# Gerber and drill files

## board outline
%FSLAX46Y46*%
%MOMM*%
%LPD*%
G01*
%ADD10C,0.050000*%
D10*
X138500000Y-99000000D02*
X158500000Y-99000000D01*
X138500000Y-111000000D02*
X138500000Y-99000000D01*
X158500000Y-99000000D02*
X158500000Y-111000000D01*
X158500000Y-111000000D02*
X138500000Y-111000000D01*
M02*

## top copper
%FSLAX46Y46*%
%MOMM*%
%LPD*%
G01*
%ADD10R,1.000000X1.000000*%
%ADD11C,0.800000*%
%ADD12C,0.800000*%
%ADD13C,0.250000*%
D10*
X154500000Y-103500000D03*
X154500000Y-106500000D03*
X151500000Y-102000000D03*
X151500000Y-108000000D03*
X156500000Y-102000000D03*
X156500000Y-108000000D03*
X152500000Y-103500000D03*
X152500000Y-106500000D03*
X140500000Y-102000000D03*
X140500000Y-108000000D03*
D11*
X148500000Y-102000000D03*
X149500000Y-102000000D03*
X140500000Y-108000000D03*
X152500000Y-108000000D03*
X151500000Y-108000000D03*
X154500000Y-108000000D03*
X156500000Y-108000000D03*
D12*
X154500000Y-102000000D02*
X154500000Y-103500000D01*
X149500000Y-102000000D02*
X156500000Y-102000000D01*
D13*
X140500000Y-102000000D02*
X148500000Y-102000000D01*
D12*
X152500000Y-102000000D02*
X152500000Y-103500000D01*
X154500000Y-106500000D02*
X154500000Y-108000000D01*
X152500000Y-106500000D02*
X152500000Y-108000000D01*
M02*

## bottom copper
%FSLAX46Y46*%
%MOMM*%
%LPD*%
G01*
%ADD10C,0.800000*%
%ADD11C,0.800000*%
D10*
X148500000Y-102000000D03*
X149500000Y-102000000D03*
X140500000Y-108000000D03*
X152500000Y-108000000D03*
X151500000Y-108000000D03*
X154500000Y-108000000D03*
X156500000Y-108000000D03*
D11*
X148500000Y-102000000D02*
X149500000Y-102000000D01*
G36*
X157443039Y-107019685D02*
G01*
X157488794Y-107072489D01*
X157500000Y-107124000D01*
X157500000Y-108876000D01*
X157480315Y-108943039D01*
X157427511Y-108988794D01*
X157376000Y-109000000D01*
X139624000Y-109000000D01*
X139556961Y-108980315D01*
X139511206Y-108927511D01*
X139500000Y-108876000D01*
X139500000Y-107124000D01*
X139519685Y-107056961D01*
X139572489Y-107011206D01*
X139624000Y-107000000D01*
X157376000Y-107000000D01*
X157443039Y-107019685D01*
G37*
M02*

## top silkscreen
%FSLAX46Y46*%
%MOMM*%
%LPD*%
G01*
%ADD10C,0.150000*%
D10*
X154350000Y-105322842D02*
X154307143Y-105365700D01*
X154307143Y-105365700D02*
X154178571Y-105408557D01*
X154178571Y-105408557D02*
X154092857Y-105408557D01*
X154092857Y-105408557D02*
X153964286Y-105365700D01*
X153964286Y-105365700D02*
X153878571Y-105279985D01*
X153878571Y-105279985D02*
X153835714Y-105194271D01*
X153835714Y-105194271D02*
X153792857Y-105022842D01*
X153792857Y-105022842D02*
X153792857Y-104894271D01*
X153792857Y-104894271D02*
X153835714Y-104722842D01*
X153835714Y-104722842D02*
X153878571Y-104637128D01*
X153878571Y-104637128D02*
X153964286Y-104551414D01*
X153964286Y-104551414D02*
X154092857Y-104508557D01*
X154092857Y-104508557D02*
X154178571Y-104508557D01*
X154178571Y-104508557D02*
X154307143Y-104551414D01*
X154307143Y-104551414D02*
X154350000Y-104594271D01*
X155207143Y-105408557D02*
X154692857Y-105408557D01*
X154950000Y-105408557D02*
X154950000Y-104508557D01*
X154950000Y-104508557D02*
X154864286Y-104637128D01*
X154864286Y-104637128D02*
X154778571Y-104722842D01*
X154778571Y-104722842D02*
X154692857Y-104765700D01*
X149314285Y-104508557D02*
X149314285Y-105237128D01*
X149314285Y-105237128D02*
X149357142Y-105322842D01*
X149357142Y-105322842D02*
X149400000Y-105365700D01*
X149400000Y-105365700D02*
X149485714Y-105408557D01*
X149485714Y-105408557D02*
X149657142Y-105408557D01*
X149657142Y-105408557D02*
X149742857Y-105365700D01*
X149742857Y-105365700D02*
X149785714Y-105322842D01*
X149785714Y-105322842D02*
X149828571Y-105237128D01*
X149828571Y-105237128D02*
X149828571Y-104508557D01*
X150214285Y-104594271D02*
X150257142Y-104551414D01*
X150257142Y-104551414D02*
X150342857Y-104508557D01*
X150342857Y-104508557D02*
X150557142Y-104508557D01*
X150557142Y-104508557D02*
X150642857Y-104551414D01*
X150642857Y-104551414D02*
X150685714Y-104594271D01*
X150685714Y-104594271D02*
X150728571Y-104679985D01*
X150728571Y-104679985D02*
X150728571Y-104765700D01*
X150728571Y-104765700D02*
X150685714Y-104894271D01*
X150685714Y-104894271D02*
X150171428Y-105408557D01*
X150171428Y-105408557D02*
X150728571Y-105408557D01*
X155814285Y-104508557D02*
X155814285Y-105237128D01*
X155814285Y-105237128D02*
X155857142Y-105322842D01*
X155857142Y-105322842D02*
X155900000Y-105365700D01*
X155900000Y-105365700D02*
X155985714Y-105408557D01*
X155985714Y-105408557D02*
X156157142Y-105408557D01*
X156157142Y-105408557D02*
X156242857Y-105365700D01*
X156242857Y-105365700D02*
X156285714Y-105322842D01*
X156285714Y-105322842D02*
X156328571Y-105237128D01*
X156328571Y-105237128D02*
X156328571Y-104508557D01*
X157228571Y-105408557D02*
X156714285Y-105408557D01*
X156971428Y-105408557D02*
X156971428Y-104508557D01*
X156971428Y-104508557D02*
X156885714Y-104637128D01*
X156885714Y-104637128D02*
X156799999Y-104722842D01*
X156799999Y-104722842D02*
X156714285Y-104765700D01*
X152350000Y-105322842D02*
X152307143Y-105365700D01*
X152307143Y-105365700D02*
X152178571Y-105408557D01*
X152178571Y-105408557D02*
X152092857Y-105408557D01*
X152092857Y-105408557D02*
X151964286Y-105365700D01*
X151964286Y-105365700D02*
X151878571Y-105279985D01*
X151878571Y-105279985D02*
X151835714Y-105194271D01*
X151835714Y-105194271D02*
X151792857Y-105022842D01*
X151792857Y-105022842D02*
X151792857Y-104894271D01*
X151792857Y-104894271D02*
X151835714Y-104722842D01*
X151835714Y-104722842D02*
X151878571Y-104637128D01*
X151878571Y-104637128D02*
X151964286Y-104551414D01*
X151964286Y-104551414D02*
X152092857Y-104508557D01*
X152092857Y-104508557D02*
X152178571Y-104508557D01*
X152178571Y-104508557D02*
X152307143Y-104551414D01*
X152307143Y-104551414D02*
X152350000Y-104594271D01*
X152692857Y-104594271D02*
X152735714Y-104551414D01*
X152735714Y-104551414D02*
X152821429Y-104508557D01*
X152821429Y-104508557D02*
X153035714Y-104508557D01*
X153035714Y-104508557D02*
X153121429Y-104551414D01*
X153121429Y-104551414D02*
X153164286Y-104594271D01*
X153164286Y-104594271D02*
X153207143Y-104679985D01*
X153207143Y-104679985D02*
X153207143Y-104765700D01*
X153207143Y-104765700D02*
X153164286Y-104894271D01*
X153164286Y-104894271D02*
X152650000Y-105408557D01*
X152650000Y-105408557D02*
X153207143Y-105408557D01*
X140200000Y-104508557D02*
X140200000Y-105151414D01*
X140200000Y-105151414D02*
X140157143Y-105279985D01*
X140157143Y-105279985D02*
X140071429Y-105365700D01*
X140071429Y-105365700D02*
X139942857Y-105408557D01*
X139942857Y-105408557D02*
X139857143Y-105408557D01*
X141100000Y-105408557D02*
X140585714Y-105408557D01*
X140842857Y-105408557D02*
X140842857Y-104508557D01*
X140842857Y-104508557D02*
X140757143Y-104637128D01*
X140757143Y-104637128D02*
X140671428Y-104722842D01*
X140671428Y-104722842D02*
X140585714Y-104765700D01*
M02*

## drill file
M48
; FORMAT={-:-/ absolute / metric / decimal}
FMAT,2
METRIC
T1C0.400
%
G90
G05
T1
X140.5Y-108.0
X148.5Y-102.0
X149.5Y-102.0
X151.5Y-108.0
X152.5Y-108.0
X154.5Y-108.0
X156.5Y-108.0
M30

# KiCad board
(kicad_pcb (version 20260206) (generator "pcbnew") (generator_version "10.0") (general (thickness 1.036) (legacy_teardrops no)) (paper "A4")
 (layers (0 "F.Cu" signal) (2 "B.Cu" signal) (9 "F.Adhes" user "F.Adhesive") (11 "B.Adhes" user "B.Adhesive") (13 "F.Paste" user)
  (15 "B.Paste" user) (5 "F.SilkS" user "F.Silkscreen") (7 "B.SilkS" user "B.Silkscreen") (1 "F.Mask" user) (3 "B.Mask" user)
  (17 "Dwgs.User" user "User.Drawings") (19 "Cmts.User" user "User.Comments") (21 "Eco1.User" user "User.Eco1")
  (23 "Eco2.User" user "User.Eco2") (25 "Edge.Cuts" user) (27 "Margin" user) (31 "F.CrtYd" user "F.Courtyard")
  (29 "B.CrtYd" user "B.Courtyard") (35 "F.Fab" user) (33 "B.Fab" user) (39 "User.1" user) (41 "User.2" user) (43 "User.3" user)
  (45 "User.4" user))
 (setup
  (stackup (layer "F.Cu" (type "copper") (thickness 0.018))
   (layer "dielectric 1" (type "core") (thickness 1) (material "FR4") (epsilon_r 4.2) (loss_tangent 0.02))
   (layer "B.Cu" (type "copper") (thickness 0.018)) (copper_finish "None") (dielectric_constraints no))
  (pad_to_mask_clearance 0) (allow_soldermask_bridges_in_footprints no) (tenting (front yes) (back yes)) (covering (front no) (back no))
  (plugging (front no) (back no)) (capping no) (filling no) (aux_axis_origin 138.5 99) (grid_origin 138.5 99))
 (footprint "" (layer "F.Cu") (at 154.5 105)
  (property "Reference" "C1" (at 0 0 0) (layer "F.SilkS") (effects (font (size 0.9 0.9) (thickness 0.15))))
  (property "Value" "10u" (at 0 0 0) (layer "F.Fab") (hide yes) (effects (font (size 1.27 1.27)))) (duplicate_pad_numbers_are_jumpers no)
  (pad "1" smd rect (at 0 -1.5) (size 1 1) (layers "F.Cu") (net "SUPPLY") (thermal_bridge_angle 45))
  (pad "2" smd rect (at 0 1.5) (size 1 1) (layers "F.Cu") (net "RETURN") (thermal_bridge_angle 45)))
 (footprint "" (layer "F.Cu") (at 151.5 105)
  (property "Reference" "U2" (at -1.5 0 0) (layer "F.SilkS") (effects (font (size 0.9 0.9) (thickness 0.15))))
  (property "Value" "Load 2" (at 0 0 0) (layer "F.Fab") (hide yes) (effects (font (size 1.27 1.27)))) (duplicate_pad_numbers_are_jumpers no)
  (pad "1" smd rect (at 0 -3) (size 1 1) (layers "F.Cu") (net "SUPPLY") (thermal_bridge_angle 45))
  (pad "2" smd rect (at 0 3) (size 1 1) (layers "F.Cu") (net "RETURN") (thermal_bridge_angle 45)))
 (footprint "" (layer "F.Cu") (at 156.5 105)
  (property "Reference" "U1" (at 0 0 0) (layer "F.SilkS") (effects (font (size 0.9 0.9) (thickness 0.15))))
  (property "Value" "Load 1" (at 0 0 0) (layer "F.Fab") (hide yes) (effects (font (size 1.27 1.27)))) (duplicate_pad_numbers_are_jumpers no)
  (pad "1" smd rect (at 0 -3) (size 1 1) (layers "F.Cu") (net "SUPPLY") (thermal_bridge_angle 45))
  (pad "2" smd rect (at 0 3) (size 1 1) (layers "F.Cu") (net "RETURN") (thermal_bridge_angle 45)))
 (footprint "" (layer "F.Cu") (at 152.5 105)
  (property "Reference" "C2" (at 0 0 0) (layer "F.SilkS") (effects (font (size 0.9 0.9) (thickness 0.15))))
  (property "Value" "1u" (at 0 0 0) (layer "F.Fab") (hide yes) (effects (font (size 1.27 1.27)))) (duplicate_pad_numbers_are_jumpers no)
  (pad "1" smd rect (at 0 -1.5) (size 1 1) (layers "F.Cu") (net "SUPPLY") (thermal_bridge_angle 45))
  (pad "2" smd rect (at 0 1.5) (size 1 1) (layers "F.Cu") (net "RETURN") (thermal_bridge_angle 45)))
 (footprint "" (layer "F.Cu") (at 140.5 105)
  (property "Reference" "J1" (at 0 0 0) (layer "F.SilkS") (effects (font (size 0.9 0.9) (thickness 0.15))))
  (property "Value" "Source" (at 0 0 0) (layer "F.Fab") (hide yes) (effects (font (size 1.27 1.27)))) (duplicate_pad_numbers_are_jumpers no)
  (pad "1" smd rect (at 0 -3) (size 1 1) (layers "F.Cu") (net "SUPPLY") (thermal_bridge_angle 45))
  (pad "2" smd rect (at 0 3) (size 1 1) (layers "F.Cu") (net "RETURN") (thermal_bridge_angle 45)))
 (gr_line (start 138.5 99) (end 158.5 99) (stroke (width 0.05) (type default)) (layer "Edge.Cuts"))
 (gr_line (start 138.5 111) (end 138.5 99) (stroke (width 0.05) (type default)) (layer "Edge.Cuts"))
 (gr_line (start 158.5 99) (end 158.5 111) (stroke (width 0.05) (type default)) (layer "Edge.Cuts"))
 (gr_line (start 158.5 111) (end 138.5 111) (stroke (width 0.05) (type default)) (layer "Edge.Cuts"))
 (segment (start 154.5 102) (end 154.5 103.5) (width 0.8) (layer "F.Cu") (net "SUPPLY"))
 (segment (start 149.5 102) (end 156.5 102) (width 0.8) (layer "F.Cu") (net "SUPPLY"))
 (segment (start 140.5 102) (end 148.5 102) (width 0.25) (layer "F.Cu") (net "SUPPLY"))
 (segment (start 152.5 102) (end 152.5 103.5) (width 0.8) (layer "F.Cu") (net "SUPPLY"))
 (via (at 148.5 102) (size 0.8) (drill 0.4) (layers "F.Cu" "B.Cu") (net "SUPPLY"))
 (via (at 149.5 102) (size 0.8) (drill 0.4) (layers "F.Cu" "B.Cu") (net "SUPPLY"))
 (segment (start 148.5 102) (end 149.5 102) (width 0.8) (layer "B.Cu") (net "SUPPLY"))
 (segment (start 154.5 106.5) (end 154.5 108) (width 0.8) (layer "F.Cu") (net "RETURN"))
 (segment (start 152.5 106.5) (end 152.5 108) (width 0.8) (layer "F.Cu") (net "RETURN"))
 (via (at 140.5 108) (size 0.8) (drill 0.4) (layers "F.Cu" "B.Cu") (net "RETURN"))
 (via (at 152.5 108) (size 0.8) (drill 0.4) (layers "F.Cu" "B.Cu") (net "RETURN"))
 (via (at 151.5 108) (size 0.8) (drill 0.4) (layers "F.Cu" "B.Cu") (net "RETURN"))
 (via (at 154.5 108) (size 0.8) (drill 0.4) (layers "F.Cu" "B.Cu") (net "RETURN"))
 (via (at 156.5 108) (size 0.8) (drill 0.4) (layers "F.Cu" "B.Cu") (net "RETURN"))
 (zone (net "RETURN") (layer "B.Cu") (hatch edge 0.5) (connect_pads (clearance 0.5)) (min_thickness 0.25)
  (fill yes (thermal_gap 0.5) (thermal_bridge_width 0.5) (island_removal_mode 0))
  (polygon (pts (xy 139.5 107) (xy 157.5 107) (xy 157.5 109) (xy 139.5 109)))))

